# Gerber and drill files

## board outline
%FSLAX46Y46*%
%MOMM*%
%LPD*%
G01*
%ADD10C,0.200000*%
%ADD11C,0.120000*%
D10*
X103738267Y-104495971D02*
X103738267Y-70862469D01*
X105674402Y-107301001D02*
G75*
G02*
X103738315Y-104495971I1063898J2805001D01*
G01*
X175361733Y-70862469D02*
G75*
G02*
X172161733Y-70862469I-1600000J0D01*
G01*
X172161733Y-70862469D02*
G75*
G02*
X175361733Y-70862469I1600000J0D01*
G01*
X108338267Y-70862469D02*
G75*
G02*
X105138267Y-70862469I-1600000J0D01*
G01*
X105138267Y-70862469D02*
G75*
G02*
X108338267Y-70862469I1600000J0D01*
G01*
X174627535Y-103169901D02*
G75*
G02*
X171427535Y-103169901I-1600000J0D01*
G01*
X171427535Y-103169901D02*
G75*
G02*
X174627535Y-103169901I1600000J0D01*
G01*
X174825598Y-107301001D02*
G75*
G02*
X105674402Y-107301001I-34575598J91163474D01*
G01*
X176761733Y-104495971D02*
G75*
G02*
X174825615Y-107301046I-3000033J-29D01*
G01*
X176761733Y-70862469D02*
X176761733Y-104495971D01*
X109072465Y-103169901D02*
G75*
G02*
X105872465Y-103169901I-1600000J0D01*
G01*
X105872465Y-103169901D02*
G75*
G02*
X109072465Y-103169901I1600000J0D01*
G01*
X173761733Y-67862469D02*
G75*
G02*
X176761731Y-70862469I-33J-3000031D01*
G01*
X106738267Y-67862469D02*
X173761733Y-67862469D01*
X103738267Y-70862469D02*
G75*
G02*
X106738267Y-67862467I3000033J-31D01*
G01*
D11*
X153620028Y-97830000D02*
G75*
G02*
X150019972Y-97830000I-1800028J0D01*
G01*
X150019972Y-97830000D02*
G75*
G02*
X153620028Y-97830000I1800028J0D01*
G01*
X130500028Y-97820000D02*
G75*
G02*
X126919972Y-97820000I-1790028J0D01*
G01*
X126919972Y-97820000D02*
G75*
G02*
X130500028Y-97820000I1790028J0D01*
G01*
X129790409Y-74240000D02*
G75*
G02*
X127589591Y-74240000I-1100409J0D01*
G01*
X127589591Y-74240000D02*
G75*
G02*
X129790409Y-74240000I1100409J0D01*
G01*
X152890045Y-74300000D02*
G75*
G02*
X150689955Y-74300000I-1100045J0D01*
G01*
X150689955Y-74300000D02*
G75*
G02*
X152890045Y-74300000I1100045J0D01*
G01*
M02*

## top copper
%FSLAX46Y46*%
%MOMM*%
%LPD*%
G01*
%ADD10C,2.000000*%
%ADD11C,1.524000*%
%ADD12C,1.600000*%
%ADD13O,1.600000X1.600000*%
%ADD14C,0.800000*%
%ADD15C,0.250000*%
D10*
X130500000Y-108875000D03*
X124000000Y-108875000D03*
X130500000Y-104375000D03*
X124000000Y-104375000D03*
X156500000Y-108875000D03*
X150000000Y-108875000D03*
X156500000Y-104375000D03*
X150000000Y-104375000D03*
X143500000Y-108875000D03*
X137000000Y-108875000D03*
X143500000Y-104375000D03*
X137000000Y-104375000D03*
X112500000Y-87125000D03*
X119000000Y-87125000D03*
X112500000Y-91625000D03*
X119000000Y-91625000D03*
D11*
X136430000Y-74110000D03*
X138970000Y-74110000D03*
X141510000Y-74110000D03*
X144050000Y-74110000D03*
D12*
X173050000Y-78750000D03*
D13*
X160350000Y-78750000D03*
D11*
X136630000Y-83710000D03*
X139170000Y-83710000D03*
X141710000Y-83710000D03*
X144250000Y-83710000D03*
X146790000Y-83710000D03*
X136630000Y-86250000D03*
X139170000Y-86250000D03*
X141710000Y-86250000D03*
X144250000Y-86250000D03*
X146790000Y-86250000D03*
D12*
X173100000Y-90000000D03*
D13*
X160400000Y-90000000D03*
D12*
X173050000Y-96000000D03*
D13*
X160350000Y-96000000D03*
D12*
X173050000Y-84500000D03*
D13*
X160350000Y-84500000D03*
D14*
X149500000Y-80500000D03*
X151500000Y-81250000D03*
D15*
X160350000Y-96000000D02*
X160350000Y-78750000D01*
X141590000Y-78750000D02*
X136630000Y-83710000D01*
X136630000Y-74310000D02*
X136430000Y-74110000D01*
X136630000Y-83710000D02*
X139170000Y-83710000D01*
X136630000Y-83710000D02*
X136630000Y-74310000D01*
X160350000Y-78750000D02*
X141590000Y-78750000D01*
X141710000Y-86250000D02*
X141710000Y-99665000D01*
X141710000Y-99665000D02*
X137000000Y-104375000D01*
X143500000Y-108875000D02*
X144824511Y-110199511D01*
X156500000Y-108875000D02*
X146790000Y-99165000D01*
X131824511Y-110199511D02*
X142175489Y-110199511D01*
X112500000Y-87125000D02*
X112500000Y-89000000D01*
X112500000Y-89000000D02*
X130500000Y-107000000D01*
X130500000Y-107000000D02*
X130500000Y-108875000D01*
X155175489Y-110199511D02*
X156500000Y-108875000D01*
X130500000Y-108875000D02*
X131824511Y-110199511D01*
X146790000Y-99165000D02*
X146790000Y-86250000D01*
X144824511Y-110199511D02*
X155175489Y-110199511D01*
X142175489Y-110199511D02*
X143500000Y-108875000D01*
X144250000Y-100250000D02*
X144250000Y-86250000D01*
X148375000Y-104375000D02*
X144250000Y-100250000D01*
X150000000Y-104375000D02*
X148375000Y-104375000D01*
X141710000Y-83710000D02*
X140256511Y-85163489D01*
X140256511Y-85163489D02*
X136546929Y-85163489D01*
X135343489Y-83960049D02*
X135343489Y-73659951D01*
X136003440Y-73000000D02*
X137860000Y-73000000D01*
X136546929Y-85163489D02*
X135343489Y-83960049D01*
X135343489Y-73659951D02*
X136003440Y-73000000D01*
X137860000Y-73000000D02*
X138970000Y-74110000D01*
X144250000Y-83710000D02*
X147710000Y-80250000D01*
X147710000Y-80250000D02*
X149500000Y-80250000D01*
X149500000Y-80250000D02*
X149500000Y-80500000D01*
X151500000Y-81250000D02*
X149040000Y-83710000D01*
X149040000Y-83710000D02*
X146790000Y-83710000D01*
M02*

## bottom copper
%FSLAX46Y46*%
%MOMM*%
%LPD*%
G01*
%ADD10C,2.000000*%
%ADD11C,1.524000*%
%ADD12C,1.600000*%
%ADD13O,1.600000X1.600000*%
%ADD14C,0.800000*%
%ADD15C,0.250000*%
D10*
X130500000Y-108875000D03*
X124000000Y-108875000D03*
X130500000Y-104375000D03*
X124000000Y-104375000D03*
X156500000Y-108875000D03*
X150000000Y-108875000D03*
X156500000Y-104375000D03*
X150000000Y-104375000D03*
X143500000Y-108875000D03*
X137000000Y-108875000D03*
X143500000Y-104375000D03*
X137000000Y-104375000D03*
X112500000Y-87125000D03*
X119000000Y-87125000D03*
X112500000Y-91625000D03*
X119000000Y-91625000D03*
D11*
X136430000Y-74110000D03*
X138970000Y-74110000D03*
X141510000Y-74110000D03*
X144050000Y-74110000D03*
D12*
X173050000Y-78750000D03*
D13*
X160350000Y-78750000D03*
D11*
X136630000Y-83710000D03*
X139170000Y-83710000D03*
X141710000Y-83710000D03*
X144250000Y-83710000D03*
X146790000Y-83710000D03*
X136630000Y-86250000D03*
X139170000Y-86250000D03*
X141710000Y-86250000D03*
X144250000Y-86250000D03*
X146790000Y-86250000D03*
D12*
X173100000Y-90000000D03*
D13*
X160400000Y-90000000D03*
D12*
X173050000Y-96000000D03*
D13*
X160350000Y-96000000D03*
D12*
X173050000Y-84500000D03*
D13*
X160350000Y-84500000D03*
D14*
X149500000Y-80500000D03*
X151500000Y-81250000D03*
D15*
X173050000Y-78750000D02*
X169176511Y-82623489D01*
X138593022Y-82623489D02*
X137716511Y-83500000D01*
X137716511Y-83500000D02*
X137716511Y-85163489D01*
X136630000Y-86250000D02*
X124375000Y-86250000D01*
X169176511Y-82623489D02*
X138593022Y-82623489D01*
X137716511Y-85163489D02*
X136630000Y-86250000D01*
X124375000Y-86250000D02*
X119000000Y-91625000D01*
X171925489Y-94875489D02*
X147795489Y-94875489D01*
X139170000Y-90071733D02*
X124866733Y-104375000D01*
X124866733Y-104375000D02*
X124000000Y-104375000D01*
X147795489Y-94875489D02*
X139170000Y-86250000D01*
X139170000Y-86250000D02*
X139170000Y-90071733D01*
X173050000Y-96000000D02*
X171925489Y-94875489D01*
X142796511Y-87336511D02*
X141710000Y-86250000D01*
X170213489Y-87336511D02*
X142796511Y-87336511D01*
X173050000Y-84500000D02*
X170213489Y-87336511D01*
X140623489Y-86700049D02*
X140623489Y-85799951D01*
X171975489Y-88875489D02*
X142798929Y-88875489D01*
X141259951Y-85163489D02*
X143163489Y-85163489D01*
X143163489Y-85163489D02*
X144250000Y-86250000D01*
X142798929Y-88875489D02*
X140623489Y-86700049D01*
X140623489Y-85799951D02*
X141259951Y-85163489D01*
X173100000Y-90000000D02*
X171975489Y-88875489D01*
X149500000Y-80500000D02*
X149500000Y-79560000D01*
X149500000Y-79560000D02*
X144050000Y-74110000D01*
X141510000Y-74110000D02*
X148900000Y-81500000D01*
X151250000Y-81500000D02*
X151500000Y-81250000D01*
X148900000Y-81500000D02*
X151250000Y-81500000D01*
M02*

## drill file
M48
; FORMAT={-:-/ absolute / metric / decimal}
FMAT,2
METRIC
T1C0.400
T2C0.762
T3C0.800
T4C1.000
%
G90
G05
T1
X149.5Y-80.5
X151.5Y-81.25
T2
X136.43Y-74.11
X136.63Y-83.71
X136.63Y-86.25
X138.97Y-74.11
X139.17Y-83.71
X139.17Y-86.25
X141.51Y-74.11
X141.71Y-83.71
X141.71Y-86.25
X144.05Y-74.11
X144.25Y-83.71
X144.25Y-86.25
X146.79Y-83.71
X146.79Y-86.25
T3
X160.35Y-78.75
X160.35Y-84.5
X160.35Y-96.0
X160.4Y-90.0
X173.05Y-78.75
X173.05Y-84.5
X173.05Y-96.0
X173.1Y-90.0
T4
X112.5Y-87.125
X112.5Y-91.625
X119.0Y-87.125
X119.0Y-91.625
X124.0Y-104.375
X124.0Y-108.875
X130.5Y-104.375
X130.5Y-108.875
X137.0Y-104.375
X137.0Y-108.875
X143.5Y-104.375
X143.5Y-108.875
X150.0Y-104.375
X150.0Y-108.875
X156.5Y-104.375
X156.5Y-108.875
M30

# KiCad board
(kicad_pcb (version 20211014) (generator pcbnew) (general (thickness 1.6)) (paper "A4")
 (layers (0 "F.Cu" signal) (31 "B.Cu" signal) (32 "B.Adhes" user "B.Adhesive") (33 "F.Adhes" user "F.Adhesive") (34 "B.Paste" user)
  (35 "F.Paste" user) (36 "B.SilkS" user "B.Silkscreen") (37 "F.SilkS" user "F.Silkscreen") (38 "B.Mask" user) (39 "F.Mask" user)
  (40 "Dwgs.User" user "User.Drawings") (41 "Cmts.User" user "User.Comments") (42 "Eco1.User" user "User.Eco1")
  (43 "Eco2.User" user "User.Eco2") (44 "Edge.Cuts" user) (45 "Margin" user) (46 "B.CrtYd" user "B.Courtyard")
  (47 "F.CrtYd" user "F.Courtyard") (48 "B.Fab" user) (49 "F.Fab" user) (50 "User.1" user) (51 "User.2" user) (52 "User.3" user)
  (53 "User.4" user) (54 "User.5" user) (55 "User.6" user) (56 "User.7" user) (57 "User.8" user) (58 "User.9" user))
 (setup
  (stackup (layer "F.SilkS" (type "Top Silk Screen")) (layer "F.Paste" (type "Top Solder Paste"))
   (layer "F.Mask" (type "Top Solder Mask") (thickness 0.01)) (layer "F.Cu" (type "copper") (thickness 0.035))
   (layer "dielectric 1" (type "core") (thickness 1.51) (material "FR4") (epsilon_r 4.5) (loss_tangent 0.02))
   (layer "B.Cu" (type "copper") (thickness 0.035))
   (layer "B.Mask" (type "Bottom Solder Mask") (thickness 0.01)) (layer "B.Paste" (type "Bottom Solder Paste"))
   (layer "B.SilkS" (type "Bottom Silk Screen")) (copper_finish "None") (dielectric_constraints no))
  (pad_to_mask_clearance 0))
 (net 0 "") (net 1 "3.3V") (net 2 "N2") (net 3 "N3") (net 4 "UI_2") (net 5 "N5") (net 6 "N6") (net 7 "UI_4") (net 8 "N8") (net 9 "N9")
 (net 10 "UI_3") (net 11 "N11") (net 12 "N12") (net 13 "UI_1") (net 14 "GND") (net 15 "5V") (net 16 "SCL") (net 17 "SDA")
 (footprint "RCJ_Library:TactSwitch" (layer "F.Cu") (at 124.5 115.875 180)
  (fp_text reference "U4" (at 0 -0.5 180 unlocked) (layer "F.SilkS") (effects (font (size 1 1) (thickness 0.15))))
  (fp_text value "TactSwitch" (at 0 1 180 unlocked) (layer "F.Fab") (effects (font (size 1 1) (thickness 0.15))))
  (pad "1" thru_hole circle (at -6 7 180) (size 2 2) (drill 1) (layers *.Cu *.Mask) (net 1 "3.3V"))
  (pad "2" thru_hole circle (at 0.5 7 180) (size 2 2) (drill 1) (layers *.Cu *.Mask) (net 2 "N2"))
  (pad "3" thru_hole circle (at -6 11.5 180) (size 2 2) (drill 1) (layers *.Cu *.Mask) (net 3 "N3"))
  (pad "4" thru_hole circle (at 0.5 11.5 180) (size 2 2) (drill 1) (layers *.Cu *.Mask) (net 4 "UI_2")))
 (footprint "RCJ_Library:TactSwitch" (layer "F.Cu") (at 150.5 115.875 180)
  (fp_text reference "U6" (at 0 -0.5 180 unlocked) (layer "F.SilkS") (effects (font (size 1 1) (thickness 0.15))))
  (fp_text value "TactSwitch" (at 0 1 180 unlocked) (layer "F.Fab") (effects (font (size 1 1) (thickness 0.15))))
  (pad "1" thru_hole circle (at -6 7 180) (size 2 2) (drill 1) (layers *.Cu *.Mask) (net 1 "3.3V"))
  (pad "2" thru_hole circle (at 0.5 7 180) (size 2 2) (drill 1) (layers *.Cu *.Mask) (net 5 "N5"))
  (pad "3" thru_hole circle (at -6 11.5 180) (size 2 2) (drill 1) (layers *.Cu *.Mask) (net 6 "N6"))
  (pad "4" thru_hole circle (at 0.5 11.5 180) (size 2 2) (drill 1) (layers *.Cu *.Mask) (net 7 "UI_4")))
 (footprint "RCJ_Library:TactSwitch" (layer "F.Cu") (at 137.5 115.875 180)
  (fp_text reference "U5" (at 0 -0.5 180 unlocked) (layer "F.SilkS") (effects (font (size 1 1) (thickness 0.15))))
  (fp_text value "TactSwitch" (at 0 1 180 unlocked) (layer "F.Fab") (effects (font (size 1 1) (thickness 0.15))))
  (pad "1" thru_hole circle (at -6 7 180) (size 2 2) (drill 1) (layers *.Cu *.Mask) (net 1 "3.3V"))
  (pad "2" thru_hole circle (at 0.5 7 180) (size 2 2) (drill 1) (layers *.Cu *.Mask) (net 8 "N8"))
  (pad "3" thru_hole circle (at -6 11.5 180) (size 2 2) (drill 1) (layers *.Cu *.Mask) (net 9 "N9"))
  (pad "4" thru_hole circle (at 0.5 11.5 180) (size 2 2) (drill 1) (layers *.Cu *.Mask) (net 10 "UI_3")))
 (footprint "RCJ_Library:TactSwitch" (layer "F.Cu") (at 118.5 80.125)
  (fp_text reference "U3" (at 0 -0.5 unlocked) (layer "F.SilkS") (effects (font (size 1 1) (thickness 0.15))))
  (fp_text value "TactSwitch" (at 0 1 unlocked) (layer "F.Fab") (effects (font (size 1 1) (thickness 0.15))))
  (pad "1" thru_hole circle (at -6 7) (size 2 2) (drill 1) (layers *.Cu *.Mask) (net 1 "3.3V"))
  (pad "2" thru_hole circle (at 0.5 7) (size 2 2) (drill 1) (layers *.Cu *.Mask) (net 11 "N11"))
  (pad "3" thru_hole circle (at -6 11.5) (size 2 2) (drill 1) (layers *.Cu *.Mask) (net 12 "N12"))
  (pad "4" thru_hole circle (at 0.5 11.5) (size 2 2) (drill 1) (layers *.Cu *.Mask) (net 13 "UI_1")))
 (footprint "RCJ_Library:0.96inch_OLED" (layer "F.Cu") (at 140.24 69.03)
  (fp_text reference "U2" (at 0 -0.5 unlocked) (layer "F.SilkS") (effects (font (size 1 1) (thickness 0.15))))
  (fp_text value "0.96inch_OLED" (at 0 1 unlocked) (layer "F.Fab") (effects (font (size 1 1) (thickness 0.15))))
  (fp_circle (center 11.58 28.8) (end 13.38 28.81) (layer "Edge.Cuts") (width 0.12) (fill none))
  (fp_circle (center -11.53 28.79) (end -9.74 28.8) (layer "Edge.Cuts") (width 0.12) (fill none))
  (fp_circle (center -11.55 5.21) (end -10.45 5.24) (layer "Edge.Cuts") (width 0.12) (fill none))
  (fp_circle (center 11.55 5.27) (end 12.65 5.28) (layer "Edge.Cuts") (width 0.12) (fill none))
  (pad "1" thru_hole circle (at -3.81 5.08) (size 1.524 1.524) (drill 0.762) (layers *.Cu *.Mask) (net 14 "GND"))
  (pad "2" thru_hole circle (at -1.27 5.08) (size 1.524 1.524) (drill 0.762) (layers *.Cu *.Mask) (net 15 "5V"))
  (pad "3" thru_hole circle (at 1.27 5.08) (size 1.524 1.524) (drill 0.762) (layers *.Cu *.Mask) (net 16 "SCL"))
  (pad "4" thru_hole circle (at 3.81 5.08) (size 1.524 1.524) (drill 0.762) (layers *.Cu *.Mask) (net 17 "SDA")))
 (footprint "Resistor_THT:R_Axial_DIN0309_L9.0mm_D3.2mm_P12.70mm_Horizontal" (layer "B.Cu") (at 173.05 78.75 180)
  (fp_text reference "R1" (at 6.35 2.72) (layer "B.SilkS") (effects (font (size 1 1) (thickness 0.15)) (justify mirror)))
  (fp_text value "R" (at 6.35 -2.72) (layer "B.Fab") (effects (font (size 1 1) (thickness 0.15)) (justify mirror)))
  (pad "1" thru_hole circle (at 0 0 180) (size 1.6 1.6) (drill 0.8) (layers *.Cu *.Mask) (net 13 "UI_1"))
  (pad "2" thru_hole oval (at 12.7 0 180) (size 1.6 1.6) (drill 0.8) (layers *.Cu *.Mask) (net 14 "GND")))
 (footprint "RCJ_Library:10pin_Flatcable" (layer "B.Cu") (at 131.55 86.25 -90)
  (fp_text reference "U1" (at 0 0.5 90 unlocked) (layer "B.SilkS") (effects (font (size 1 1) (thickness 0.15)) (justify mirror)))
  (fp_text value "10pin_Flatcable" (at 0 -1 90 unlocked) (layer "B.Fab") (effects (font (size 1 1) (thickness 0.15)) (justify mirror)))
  (pad "1" thru_hole circle (at -2.54 -5.08 270) (size 1.524 1.524) (drill 0.762) (layers *.Cu *.Mask) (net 14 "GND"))
  (pad "2" thru_hole circle (at -2.54 -7.62 270) (size 1.524 1.524) (drill 0.762) (layers *.Cu *.Mask) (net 14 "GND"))
  (pad "3" thru_hole circle (at -2.54 -10.16 270) (size 1.524 1.524) (drill 0.762) (layers *.Cu *.Mask) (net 15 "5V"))
  (pad "4" thru_hole circle (at -2.54 -12.7 270) (size 1.524 1.524) (drill 0.762) (layers *.Cu *.Mask) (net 17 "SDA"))
  (pad "5" thru_hole circle (at -2.54 -15.24 270) (size 1.524 1.524) (drill 0.762) (layers *.Cu *.Mask) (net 16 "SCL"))
  (pad "6" thru_hole circle (at 0 -5.08 270) (size 1.524 1.524) (drill 0.762) (layers *.Cu *.Mask) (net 13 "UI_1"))
  (pad "7" thru_hole circle (at 0 -7.62 270) (size 1.524 1.524) (drill 0.762) (layers *.Cu *.Mask) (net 4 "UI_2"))
  (pad "8" thru_hole circle (at 0 -10.16 270) (size 1.524 1.524) (drill 0.762) (layers *.Cu *.Mask) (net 10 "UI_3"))
  (pad "9" thru_hole circle (at 0 -12.7 270) (size 1.524 1.524) (drill 0.762) (layers *.Cu *.Mask) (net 7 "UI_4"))
  (pad "10" thru_hole circle (at 0 -15.24 270) (size 1.524 1.524) (drill 0.762) (layers *.Cu *.Mask) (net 1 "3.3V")))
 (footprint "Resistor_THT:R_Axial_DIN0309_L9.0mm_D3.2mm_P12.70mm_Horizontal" (layer "B.Cu") (at 173.1 90 180)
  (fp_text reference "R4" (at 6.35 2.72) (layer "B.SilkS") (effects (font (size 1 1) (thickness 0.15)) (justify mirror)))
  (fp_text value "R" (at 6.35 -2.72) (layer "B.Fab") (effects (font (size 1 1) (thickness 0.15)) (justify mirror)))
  (pad "1" thru_hole circle (at 0 0 180) (size 1.6 1.6) (drill 0.8) (layers *.Cu *.Mask) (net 7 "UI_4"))
  (pad "2" thru_hole oval (at 12.7 0 180) (size 1.6 1.6) (drill 0.8) (layers *.Cu *.Mask) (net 14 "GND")))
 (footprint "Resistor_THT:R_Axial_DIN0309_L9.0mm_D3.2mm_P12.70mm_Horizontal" (layer "B.Cu") (at 173.05 96 180)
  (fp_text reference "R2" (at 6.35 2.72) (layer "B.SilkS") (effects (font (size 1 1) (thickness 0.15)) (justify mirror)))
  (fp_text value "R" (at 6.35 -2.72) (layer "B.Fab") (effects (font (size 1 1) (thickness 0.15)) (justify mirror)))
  (pad "1" thru_hole circle (at 0 0 180) (size 1.6 1.6) (drill 0.8) (layers *.Cu *.Mask) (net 4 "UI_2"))
  (pad "2" thru_hole oval (at 12.7 0 180) (size 1.6 1.6) (drill 0.8) (layers *.Cu *.Mask) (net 14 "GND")))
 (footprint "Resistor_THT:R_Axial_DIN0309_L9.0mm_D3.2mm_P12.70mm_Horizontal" (layer "B.Cu") (at 173.05 84.5 180)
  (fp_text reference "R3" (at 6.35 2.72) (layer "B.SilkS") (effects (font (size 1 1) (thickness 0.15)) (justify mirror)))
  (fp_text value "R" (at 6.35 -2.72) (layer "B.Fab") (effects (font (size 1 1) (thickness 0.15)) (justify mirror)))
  (pad "1" thru_hole circle (at 0 0 180) (size 1.6 1.6) (drill 0.8) (layers *.Cu *.Mask) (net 10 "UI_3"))
  (pad "2" thru_hole oval (at 12.7 0 180) (size 1.6 1.6) (drill 0.8) (layers *.Cu *.Mask) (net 14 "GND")))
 (gr_line (start 103.738267 104.495971) (end 103.738267 70.862469) (layer "Edge.Cuts") (width 0.2))
 (gr_arc (start 105.674402 107.301001) (mid 104.2693 106.200143) (end 103.738267 104.495971) (layer "Edge.Cuts") (width 0.2))
 (gr_circle (center 173.761733 70.862469) (end 175.361733 70.862469) (layer "Edge.Cuts") (width 0.2) (fill none))
 (gr_circle (center 106.738267 70.862469) (end 108.338267 70.862469) (layer "Edge.Cuts") (width 0.2) (fill none))
 (gr_circle (center 173.027535 103.169901) (end 174.627535 103.169901) (layer "Edge.Cuts") (width 0.2) (fill none))
 (gr_arc (start 174.825598 107.301001) (mid 140.25 113.637532) (end 105.674402 107.301001) (layer "Edge.Cuts") (width 0.2))
 (gr_arc (start 176.761733 104.495971) (mid 176.2307 106.200143) (end 174.825598 107.301001) (layer "Edge.Cuts") (width 0.2))
 (gr_line (start 176.761733 70.862469) (end 176.761733 104.495971) (layer "Edge.Cuts") (width 0.2))
 (gr_circle (center 107.472465 103.169901) (end 109.072465 103.169901) (layer "Edge.Cuts") (width 0.2) (fill none))
 (gr_arc (start 173.761733 67.862469) (mid 175.883054 68.741148) (end 176.761733 70.862469) (layer "Edge.Cuts") (width 0.2))
 (gr_line (start 106.738267 67.862469) (end 173.761733 67.862469) (layer "Edge.Cuts") (width 0.2))
 (gr_arc (start 103.738267 70.862469) (mid 104.616946 68.741148) (end 106.738267 67.862469) (layer "Edge.Cuts") (width 0.2))
 (segment (start 173.05 78.75) (end 169.176511 82.623489) (width 0.25) (layer "B.Cu") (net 13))
 (segment (start 138.593022 82.623489) (end 137.716511 83.5) (width 0.25) (layer "B.Cu") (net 13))
 (segment (start 137.716511 83.5) (end 137.716511 85.163489) (width 0.25) (layer "B.Cu") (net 13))
 (segment (start 136.63 86.25) (end 124.375 86.25) (width 0.25) (layer "B.Cu") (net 13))
 (segment (start 169.176511 82.623489) (end 138.593022 82.623489) (width 0.25) (layer "B.Cu") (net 13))
 (segment (start 137.716511 85.163489) (end 136.63 86.25) (width 0.25) (layer "B.Cu") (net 13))
 (segment (start 124.375 86.25) (end 119 91.625) (width 0.25) (layer "B.Cu") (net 13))
 (segment (start 160.35 96) (end 160.35 78.75) (width 0.25) (layer "F.Cu") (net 14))
 (segment (start 141.59 78.75) (end 136.63 83.71) (width 0.25) (layer "F.Cu") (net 14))
 (segment (start 136.63 74.31) (end 136.43 74.11) (width 0.25) (layer "F.Cu") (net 14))
 (segment (start 136.63 83.71) (end 139.17 83.71) (width 0.25) (layer "F.Cu") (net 14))
 (segment (start 136.63 83.71) (end 136.63 74.31) (width 0.25) (layer "F.Cu") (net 14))
 (segment (start 160.35 78.75) (end 141.59 78.75) (width 0.25) (layer "F.Cu") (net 14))
 (segment (start 171.925489 94.875489) (end 147.795489 94.875489) (width 0.25) (layer "B.Cu") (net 4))
 (segment (start 139.17 90.071733) (end 124.866733 104.375) (width 0.25) (layer "B.Cu") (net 4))
 (segment (start 124.866733 104.375) (end 124 104.375) (width 0.25) (layer "B.Cu") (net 4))
 (segment (start 147.795489 94.875489) (end 139.17 86.25) (width 0.25) (layer "B.Cu") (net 4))
 (segment (start 139.17 86.25) (end 139.17 90.071733) (width 0.25) (layer "B.Cu") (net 4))
 (segment (start 173.05 96) (end 171.925489 94.875489) (width 0.25) (layer "B.Cu") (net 4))
 (segment (start 141.71 86.25) (end 141.71 99.665) (width 0.25) (layer "F.Cu") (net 10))
 (segment (start 141.71 99.665) (end 137 104.375) (width 0.25) (layer "F.Cu") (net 10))
 (segment (start 142.796511 87.336511) (end 141.71 86.25) (width 0.25) (layer "B.Cu") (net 10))
 (segment (start 170.213489 87.336511) (end 142.796511 87.336511) (width 0.25) (layer "B.Cu") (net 10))
 (segment (start 173.05 84.5) (end 170.213489 87.336511) (width 0.25) (layer "B.Cu") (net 10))
 (segment (start 143.5 108.875) (end 144.824511 110.199511) (width 0.25) (layer "F.Cu") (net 1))
 (segment (start 156.5 108.875) (end 146.79 99.165) (width 0.25) (layer "F.Cu") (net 1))
 (segment (start 131.824511 110.199511) (end 142.175489 110.199511) (width 0.25) (layer "F.Cu") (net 1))
 (segment (start 112.5 87.125) (end 112.5 89) (width 0.25) (layer "F.Cu") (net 1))
 (segment (start 112.5 89) (end 130.5 107) (width 0.25) (layer "F.Cu") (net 1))
 (segment (start 130.5 107) (end 130.5 108.875) (width 0.25) (layer "F.Cu") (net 1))
 (segment (start 155.175489 110.199511) (end 156.5 108.875) (width 0.25) (layer "F.Cu") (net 1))
 (segment (start 130.5 108.875) (end 131.824511 110.199511) (width 0.25) (layer "F.Cu") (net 1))
 (segment (start 146.79 99.165) (end 146.79 86.25) (width 0.25) (layer "F.Cu") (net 1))
 (segment (start 144.824511 110.199511) (end 155.175489 110.199511) (width 0.25) (layer "F.Cu") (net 1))
 (segment (start 142.175489 110.199511) (end 143.5 108.875) (width 0.25) (layer "F.Cu") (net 1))
 (segment (start 144.25 100.25) (end 144.25 86.25) (width 0.25) (layer "F.Cu") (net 7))
 (segment (start 148.375 104.375) (end 144.25 100.25) (width 0.25) (layer "F.Cu") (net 7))
 (segment (start 150 104.375) (end 148.375 104.375) (width 0.25) (layer "F.Cu") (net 7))
 (segment (start 140.623489 86.700049) (end 140.623489 85.799951) (width 0.25) (layer "B.Cu") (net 7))
 (segment (start 171.975489 88.875489) (end 142.798929 88.875489) (width 0.25) (layer "B.Cu") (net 7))
 (segment (start 141.259951 85.163489) (end 143.163489 85.163489) (width 0.25) (layer "B.Cu") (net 7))
 (segment (start 143.163489 85.163489) (end 144.25 86.25) (width 0.25) (layer "B.Cu") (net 7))
 (segment (start 142.798929 88.875489) (end 140.623489 86.700049) (width 0.25) (layer "B.Cu") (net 7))
 (segment (start 140.623489 85.799951) (end 141.259951 85.163489) (width 0.25) (layer "B.Cu") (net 7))
 (segment (start 173.1 90) (end 171.975489 88.875489) (width 0.25) (layer "B.Cu") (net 7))
 (segment (start 141.71 83.71) (end 140.256511 85.163489) (width 0.25) (layer "F.Cu") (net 15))
 (segment (start 140.256511 85.163489) (end 136.546929 85.163489) (width 0.25) (layer "F.Cu") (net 15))
 (segment (start 135.343489 83.960049) (end 135.343489 73.659951) (width 0.25) (layer "F.Cu") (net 15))
 (segment (start 136.00344 73) (end 137.86 73) (width 0.25) (layer "F.Cu") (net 15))
 (segment (start 136.546929 85.163489) (end 135.343489 83.960049) (width 0.25) (layer "F.Cu") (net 15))
 (segment (start 135.343489 73.659951) (end 136.00344 73) (width 0.25) (layer "F.Cu") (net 15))
 (segment (start 137.86 73) (end 138.97 74.11) (width 0.25) (layer "F.Cu") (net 15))
 (segment (start 144.25 83.71) (end 147.71 80.25) (width 0.25) (layer "F.Cu") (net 17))
 (segment (start 147.71 80.25) (end 149.5 80.25) (width 0.25) (layer "F.Cu") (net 17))
 (segment (start 149.5 80.25) (end 149.5 80.5) (width 0.25) (layer "F.Cu") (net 17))
 (via (at 149.5 80.5) (size 0.8) (drill 0.4) (layers "F.Cu" "B.Cu") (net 17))
 (segment (start 149.5 80.5) (end 149.5 79.56) (width 0.25) (layer "B.Cu") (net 17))
 (segment (start 149.5 79.56) (end 144.05 74.11) (width 0.25) (layer "B.Cu") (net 17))
 (segment (start 151.5 81.25) (end 149.04 83.71) (width 0.25) (layer "F.Cu") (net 16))
 (segment (start 149.04 83.71) (end 146.79 83.71) (width 0.25) (layer "F.Cu") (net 16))
 (via (at 151.5 81.25) (size 0.8) (drill 0.4) (layers "F.Cu" "B.Cu") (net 16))
 (segment (start 141.51 74.11) (end 148.9 81.5) (width 0.25) (layer "B.Cu") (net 16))
 (segment (start 151.25 81.5) (end 151.5 81.25) (width 0.25) (layer "B.Cu") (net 16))
 (segment (start 148.9 81.5) (end 151.25 81.5) (width 0.25) (layer "B.Cu") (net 16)))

